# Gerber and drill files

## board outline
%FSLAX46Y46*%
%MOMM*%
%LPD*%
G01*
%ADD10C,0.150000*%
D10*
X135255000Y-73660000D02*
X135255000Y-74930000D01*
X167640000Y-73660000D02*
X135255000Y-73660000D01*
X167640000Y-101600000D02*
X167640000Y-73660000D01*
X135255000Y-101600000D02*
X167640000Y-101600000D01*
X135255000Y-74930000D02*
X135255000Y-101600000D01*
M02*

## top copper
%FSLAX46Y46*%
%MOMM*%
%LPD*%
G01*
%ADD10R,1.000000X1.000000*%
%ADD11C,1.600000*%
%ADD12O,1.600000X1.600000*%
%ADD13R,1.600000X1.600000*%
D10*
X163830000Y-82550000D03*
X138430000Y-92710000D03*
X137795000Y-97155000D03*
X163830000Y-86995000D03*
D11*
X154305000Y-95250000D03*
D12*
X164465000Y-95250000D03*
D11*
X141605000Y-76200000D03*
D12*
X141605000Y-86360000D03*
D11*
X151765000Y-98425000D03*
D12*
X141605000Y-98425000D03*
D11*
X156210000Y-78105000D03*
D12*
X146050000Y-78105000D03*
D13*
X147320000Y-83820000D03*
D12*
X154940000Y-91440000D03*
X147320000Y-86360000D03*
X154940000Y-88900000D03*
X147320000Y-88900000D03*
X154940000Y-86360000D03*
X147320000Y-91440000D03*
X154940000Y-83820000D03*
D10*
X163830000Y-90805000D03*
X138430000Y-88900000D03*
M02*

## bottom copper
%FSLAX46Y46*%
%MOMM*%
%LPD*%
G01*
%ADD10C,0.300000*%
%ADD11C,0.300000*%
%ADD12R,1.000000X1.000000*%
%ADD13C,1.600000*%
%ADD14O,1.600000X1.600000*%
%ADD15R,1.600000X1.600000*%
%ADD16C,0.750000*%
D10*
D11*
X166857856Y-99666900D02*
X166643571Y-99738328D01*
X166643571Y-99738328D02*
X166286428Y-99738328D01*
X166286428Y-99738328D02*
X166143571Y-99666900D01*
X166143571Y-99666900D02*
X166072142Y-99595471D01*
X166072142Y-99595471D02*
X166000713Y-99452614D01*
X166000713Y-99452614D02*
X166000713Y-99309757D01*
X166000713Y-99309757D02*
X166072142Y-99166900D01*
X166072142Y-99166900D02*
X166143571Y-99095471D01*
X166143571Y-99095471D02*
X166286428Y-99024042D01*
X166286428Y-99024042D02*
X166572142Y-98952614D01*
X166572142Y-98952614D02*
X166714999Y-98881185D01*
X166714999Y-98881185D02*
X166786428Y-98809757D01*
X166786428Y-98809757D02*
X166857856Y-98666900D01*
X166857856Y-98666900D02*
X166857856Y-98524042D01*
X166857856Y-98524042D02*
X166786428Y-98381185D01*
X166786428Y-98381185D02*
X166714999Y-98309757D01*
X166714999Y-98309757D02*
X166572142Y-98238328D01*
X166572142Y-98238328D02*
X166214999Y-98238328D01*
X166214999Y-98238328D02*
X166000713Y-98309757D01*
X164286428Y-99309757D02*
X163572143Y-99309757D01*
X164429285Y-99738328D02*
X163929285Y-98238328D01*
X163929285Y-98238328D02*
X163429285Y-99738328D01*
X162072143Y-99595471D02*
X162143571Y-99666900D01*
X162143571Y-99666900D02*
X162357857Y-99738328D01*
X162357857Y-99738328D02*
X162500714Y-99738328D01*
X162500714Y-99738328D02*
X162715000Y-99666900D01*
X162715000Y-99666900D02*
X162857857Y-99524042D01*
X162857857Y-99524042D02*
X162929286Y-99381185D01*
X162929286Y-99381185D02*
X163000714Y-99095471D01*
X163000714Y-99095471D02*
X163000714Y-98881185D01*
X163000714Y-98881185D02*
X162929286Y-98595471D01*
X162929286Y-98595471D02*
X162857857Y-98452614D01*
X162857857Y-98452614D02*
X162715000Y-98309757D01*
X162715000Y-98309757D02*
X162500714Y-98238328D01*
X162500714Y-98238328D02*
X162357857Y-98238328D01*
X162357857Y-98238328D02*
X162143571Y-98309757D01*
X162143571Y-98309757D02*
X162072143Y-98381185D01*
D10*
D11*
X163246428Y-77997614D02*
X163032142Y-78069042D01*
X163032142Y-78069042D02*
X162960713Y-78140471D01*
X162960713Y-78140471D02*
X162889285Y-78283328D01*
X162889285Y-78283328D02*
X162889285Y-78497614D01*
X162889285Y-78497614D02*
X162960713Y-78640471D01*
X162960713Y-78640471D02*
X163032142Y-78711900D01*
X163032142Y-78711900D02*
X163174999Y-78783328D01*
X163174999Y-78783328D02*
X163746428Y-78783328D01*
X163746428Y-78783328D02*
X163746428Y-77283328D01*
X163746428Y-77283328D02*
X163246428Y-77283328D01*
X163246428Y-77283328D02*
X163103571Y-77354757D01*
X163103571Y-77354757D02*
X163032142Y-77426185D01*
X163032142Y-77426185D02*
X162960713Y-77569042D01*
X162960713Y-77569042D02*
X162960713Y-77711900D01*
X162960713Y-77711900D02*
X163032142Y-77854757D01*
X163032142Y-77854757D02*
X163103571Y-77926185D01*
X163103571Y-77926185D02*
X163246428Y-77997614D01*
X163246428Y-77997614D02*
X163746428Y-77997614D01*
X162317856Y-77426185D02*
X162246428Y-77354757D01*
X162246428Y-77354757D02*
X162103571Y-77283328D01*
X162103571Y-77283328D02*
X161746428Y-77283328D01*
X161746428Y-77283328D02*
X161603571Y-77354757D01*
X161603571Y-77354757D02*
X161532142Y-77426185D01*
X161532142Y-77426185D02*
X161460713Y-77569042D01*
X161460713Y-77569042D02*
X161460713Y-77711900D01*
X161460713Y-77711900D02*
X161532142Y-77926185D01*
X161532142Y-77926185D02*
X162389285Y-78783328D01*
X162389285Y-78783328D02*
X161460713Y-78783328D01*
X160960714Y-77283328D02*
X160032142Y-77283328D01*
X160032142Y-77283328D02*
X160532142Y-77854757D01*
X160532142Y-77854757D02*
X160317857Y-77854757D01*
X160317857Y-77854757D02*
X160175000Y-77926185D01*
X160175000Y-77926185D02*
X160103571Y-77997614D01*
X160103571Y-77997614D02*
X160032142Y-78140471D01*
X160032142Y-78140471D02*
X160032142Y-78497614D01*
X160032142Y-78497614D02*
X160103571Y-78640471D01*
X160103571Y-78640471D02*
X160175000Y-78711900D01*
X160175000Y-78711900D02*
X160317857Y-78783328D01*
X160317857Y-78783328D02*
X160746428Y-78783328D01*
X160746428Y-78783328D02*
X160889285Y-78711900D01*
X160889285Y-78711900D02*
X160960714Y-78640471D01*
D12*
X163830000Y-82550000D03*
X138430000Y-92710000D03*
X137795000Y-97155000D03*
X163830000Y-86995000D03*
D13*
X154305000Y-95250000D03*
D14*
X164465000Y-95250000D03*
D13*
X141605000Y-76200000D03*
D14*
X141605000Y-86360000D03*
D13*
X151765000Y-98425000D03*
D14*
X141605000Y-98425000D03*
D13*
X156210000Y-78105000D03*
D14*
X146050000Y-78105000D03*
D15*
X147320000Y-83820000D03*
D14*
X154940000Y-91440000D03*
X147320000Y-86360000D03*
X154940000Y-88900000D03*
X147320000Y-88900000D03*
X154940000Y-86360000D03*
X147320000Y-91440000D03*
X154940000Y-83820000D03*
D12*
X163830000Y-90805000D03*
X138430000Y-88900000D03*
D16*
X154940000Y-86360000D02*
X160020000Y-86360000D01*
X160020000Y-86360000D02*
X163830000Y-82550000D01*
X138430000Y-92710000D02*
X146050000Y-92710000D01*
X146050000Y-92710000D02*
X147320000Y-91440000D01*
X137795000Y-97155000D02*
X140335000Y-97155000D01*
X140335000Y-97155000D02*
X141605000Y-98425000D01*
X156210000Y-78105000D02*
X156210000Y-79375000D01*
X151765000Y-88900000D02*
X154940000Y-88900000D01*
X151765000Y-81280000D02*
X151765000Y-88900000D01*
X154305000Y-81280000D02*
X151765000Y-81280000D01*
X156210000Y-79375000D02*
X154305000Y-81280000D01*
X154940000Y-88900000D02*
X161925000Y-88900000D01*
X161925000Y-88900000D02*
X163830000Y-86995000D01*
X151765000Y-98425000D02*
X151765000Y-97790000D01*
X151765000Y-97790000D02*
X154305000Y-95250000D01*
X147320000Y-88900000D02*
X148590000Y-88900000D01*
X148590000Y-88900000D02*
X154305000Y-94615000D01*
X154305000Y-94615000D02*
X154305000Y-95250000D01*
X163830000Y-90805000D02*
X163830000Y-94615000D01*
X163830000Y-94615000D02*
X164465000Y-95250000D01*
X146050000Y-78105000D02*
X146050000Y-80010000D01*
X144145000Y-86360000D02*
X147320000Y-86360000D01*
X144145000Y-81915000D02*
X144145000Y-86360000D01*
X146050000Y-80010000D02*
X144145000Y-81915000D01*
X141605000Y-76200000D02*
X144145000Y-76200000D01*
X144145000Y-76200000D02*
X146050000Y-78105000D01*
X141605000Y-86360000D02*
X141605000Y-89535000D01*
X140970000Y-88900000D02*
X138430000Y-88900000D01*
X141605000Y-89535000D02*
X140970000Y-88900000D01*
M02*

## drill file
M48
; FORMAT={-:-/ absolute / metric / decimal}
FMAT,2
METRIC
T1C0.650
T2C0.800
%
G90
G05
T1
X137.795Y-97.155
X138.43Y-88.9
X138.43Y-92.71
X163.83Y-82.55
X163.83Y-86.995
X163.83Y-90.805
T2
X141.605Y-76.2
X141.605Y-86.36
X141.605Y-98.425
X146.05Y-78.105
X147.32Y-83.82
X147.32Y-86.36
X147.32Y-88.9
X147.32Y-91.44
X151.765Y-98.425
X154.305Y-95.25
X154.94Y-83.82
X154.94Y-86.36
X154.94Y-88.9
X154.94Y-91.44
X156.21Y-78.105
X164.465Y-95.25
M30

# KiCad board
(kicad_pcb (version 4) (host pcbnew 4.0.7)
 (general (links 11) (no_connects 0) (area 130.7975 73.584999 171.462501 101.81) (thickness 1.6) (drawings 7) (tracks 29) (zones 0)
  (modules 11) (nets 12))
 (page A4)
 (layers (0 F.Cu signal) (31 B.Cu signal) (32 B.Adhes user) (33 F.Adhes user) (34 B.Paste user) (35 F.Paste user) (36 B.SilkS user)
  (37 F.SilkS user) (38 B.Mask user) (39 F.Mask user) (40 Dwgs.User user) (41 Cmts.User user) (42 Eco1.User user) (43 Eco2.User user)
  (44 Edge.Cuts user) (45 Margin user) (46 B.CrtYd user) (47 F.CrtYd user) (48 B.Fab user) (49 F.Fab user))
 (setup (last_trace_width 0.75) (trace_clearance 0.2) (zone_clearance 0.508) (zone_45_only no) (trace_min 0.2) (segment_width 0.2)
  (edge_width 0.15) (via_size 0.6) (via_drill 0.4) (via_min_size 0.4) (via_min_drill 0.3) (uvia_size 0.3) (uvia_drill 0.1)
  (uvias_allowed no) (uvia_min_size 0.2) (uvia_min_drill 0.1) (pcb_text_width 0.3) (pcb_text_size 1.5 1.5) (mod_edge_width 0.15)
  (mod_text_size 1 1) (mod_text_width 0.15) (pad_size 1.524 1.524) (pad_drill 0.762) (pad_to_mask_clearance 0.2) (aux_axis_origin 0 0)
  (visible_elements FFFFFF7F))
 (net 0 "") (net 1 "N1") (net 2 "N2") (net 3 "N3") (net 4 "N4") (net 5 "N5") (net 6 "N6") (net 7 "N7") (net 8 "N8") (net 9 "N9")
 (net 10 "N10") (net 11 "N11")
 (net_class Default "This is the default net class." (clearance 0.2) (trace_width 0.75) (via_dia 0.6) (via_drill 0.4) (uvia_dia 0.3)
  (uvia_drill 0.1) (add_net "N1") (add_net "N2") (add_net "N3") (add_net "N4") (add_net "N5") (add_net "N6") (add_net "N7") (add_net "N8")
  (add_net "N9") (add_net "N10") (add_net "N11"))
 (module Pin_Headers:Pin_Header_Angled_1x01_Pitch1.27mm (layer F.Cu) (at 163.83 82.55)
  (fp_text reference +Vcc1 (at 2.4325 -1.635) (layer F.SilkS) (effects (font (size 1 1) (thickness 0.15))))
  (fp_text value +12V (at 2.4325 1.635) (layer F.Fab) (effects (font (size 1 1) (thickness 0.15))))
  (pad 1 thru_hole rect (at 0 0) (size 1 1) (drill 0.65) (layers *.Cu *.Mask) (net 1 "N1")))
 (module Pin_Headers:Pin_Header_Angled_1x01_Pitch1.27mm (layer F.Cu) (at 138.43 92.71 180)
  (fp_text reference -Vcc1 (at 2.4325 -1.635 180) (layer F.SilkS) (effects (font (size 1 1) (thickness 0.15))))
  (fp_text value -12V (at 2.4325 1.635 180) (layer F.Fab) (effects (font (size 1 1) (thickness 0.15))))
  (pad 1 thru_hole rect (at 0 0 180) (size 1 1) (drill 0.65) (layers *.Cu *.Mask) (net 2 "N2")))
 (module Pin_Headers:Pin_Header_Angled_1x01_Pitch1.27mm (layer F.Cu) (at 137.795 97.155 180)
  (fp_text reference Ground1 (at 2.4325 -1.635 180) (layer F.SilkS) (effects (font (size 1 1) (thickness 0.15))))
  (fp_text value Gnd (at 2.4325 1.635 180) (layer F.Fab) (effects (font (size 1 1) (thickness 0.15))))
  (pad 1 thru_hole rect (at 0 0 180) (size 1 1) (drill 0.65) (layers *.Cu *.Mask) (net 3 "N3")))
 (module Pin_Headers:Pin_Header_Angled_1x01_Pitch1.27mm (layer F.Cu) (at 163.83 86.995)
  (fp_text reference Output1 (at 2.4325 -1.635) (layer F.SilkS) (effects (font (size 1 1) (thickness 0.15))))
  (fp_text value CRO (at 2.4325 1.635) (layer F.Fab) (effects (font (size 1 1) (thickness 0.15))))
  (pad 1 thru_hole rect (at 0 0) (size 1 1) (drill 0.65) (layers *.Cu *.Mask) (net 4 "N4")))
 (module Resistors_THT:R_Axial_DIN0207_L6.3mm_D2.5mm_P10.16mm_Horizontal (layer F.Cu) (at 154.305 95.25)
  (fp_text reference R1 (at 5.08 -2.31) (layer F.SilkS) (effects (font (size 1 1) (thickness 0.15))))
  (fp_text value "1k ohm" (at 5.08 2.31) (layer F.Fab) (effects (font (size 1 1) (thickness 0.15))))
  (pad 1 thru_hole circle (at 0 0) (size 1.6 1.6) (drill 0.8) (layers *.Cu *.Mask) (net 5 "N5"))
  (pad 2 thru_hole oval (at 10.16 0) (size 1.6 1.6) (drill 0.8) (layers *.Cu *.Mask) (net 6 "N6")))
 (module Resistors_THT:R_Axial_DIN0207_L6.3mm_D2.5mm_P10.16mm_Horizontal (layer F.Cu) (at 141.605 76.2 270)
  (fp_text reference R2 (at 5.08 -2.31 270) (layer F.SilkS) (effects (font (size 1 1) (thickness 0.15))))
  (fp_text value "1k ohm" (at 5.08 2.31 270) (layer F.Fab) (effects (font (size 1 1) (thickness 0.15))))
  (pad 1 thru_hole circle (at 0 0 270) (size 1.6 1.6) (drill 0.8) (layers *.Cu *.Mask) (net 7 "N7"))
  (pad 2 thru_hole oval (at 10.16 0 270) (size 1.6 1.6) (drill 0.8) (layers *.Cu *.Mask) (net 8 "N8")))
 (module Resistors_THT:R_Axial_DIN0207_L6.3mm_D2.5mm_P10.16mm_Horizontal (layer F.Cu) (at 151.765 98.425 180)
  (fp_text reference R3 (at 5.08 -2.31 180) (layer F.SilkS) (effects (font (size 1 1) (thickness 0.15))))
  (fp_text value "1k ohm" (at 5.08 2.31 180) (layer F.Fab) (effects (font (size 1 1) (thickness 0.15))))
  (pad 1 thru_hole circle (at 0 0 180) (size 1.6 1.6) (drill 0.8) (layers *.Cu *.Mask) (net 5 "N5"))
  (pad 2 thru_hole oval (at 10.16 0 180) (size 1.6 1.6) (drill 0.8) (layers *.Cu *.Mask) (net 3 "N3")))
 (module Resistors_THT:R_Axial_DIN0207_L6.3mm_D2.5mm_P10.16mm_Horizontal (layer F.Cu) (at 156.21 78.105 180)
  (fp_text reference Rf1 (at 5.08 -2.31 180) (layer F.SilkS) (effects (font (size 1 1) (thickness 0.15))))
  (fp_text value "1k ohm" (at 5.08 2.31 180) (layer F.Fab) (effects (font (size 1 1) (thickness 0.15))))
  (pad 1 thru_hole circle (at 0 0 180) (size 1.6 1.6) (drill 0.8) (layers *.Cu *.Mask) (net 4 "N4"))
  (pad 2 thru_hole oval (at 10.16 0 180) (size 1.6 1.6) (drill 0.8) (layers *.Cu *.Mask) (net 7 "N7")))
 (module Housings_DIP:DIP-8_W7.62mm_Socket (layer F.Cu) (at 147.32 83.82)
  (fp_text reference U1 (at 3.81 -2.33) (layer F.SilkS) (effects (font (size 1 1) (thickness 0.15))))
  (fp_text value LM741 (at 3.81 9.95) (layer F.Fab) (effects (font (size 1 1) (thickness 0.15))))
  (pad 1 thru_hole rect (at 0 0) (size 1.6 1.6) (drill 0.8) (layers *.Cu *.Mask) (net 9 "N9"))
  (pad 5 thru_hole oval (at 7.62 7.62) (size 1.6 1.6) (drill 0.8) (layers *.Cu *.Mask) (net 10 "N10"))
  (pad 2 thru_hole oval (at 0 2.54) (size 1.6 1.6) (drill 0.8) (layers *.Cu *.Mask) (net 7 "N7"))
  (pad 6 thru_hole oval (at 7.62 5.08) (size 1.6 1.6) (drill 0.8) (layers *.Cu *.Mask) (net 4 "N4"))
  (pad 3 thru_hole oval (at 0 5.08) (size 1.6 1.6) (drill 0.8) (layers *.Cu *.Mask) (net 5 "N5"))
  (pad 7 thru_hole oval (at 7.62 2.54) (size 1.6 1.6) (drill 0.8) (layers *.Cu *.Mask) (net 1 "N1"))
  (pad 4 thru_hole oval (at 0 7.62) (size 1.6 1.6) (drill 0.8) (layers *.Cu *.Mask) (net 2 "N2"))
  (pad 8 thru_hole oval (at 7.62 0) (size 1.6 1.6) (drill 0.8) (layers *.Cu *.Mask) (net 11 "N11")))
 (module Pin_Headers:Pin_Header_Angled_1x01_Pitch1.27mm (layer F.Cu) (at 163.83 90.805)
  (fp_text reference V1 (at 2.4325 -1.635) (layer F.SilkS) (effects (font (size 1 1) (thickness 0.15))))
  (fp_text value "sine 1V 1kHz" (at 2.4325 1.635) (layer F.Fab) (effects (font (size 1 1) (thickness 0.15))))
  (pad 1 thru_hole rect (at 0 0) (size 1 1) (drill 0.65) (layers *.Cu *.Mask) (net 6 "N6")))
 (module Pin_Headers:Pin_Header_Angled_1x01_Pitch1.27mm (layer F.Cu) (at 138.43 88.9 180)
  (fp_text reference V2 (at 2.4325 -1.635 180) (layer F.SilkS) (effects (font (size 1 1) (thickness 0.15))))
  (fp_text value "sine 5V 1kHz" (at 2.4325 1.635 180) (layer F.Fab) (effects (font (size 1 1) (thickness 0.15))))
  (pad 1 thru_hole rect (at 0 0 180) (size 1 1) (drill 0.65) (layers *.Cu *.Mask) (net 8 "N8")))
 (gr_line (start 135.255 73.66) (end 135.255 74.93) (angle 90) (layer Edge.Cuts) (width 0.15))
 (gr_line (start 167.64 73.66) (end 135.255 73.66) (angle 90) (layer Edge.Cuts) (width 0.15))
 (gr_line (start 167.64 101.6) (end 167.64 73.66) (angle 90) (layer Edge.Cuts) (width 0.15))
 (gr_line (start 135.255 101.6) (end 167.64 101.6) (angle 90) (layer Edge.Cuts) (width 0.15))
 (gr_line (start 135.255 74.93) (end 135.255 101.6) (angle 90) (layer Edge.Cuts) (width 0.15))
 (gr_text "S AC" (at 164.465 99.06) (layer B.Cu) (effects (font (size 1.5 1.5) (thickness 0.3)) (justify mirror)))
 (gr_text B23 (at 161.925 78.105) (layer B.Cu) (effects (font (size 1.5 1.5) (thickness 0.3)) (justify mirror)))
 (segment (start 154.94 86.36) (end 160.02 86.36) (width 0.75) (layer B.Cu) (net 1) (status 400000))
 (segment (start 160.02 86.36) (end 163.83 82.55) (width 0.75) (layer B.Cu) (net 1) (status 800000))
 (segment (start 138.43 92.71) (end 146.05 92.71) (width 0.75) (layer B.Cu) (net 2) (status 400000))
 (segment (start 146.05 92.71) (end 147.32 91.44) (width 0.75) (layer B.Cu) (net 2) (status 800000))
 (segment (start 137.795 97.155) (end 140.335 97.155) (width 0.75) (layer B.Cu) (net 3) (status 400000))
 (segment (start 140.335 97.155) (end 141.605 98.425) (width 0.75) (layer B.Cu) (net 3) (status 800000))
 (segment (start 156.21 78.105) (end 156.21 79.375) (width 0.75) (layer B.Cu) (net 4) (status 400000))
 (segment (start 151.765 88.9) (end 154.94 88.9) (width 0.75) (layer B.Cu) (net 4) (status 800000))
 (segment (start 151.765 81.28) (end 151.765 88.9) (width 0.75) (layer B.Cu) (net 4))
 (segment (start 154.305 81.28) (end 151.765 81.28) (width 0.75) (layer B.Cu) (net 4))
 (segment (start 156.21 79.375) (end 154.305 81.28) (width 0.75) (layer B.Cu) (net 4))
 (segment (start 154.94 88.9) (end 161.925 88.9) (width 0.75) (layer B.Cu) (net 4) (status 400000))
 (segment (start 161.925 88.9) (end 163.83 86.995) (width 0.75) (layer B.Cu) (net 4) (status 800000))
 (segment (start 151.765 98.425) (end 151.765 97.79) (width 0.75) (layer B.Cu) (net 5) (status C00000))
 (segment (start 151.765 97.79) (end 154.305 95.25) (width 0.75) (layer B.Cu) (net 5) (status C00000))
 (segment (start 147.32 88.9) (end 148.59 88.9) (width 0.75) (layer B.Cu) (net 5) (status 400000))
 (segment (start 148.59 88.9) (end 154.305 94.615) (width 0.75) (layer B.Cu) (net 5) (status 800000))
 (segment (start 154.305 94.615) (end 154.305 95.25) (width 0.75) (layer B.Cu) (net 5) (status C00000))
 (segment (start 163.83 90.805) (end 163.83 94.615) (width 0.75) (layer B.Cu) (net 6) (status 400000))
 (segment (start 163.83 94.615) (end 164.465 95.25) (width 0.75) (layer B.Cu) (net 6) (status 800000))
 (segment (start 146.05 78.105) (end 146.05 80.01) (width 0.75) (layer B.Cu) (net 7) (status 400000))
 (segment (start 144.145 86.36) (end 147.32 86.36) (width 0.75) (layer B.Cu) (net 7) (status 800000))
 (segment (start 144.145 81.915) (end 144.145 86.36) (width 0.75) (layer B.Cu) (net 7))
 (segment (start 146.05 80.01) (end 144.145 81.915) (width 0.75) (layer B.Cu) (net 7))
 (segment (start 141.605 76.2) (end 144.145 76.2) (width 0.75) (layer B.Cu) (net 7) (status 400000))
 (segment (start 144.145 76.2) (end 146.05 78.105) (width 0.75) (layer B.Cu) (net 7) (status 800000))
 (segment (start 141.605 86.36) (end 141.605 89.535) (width 0.75) (layer B.Cu) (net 8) (status 400000))
 (segment (start 140.97 88.9) (end 138.43 88.9) (width 0.75) (layer B.Cu) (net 8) (status 800000))
 (segment (start 141.605 89.535) (end 140.97 88.9) (width 0.75) (layer B.Cu) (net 8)))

